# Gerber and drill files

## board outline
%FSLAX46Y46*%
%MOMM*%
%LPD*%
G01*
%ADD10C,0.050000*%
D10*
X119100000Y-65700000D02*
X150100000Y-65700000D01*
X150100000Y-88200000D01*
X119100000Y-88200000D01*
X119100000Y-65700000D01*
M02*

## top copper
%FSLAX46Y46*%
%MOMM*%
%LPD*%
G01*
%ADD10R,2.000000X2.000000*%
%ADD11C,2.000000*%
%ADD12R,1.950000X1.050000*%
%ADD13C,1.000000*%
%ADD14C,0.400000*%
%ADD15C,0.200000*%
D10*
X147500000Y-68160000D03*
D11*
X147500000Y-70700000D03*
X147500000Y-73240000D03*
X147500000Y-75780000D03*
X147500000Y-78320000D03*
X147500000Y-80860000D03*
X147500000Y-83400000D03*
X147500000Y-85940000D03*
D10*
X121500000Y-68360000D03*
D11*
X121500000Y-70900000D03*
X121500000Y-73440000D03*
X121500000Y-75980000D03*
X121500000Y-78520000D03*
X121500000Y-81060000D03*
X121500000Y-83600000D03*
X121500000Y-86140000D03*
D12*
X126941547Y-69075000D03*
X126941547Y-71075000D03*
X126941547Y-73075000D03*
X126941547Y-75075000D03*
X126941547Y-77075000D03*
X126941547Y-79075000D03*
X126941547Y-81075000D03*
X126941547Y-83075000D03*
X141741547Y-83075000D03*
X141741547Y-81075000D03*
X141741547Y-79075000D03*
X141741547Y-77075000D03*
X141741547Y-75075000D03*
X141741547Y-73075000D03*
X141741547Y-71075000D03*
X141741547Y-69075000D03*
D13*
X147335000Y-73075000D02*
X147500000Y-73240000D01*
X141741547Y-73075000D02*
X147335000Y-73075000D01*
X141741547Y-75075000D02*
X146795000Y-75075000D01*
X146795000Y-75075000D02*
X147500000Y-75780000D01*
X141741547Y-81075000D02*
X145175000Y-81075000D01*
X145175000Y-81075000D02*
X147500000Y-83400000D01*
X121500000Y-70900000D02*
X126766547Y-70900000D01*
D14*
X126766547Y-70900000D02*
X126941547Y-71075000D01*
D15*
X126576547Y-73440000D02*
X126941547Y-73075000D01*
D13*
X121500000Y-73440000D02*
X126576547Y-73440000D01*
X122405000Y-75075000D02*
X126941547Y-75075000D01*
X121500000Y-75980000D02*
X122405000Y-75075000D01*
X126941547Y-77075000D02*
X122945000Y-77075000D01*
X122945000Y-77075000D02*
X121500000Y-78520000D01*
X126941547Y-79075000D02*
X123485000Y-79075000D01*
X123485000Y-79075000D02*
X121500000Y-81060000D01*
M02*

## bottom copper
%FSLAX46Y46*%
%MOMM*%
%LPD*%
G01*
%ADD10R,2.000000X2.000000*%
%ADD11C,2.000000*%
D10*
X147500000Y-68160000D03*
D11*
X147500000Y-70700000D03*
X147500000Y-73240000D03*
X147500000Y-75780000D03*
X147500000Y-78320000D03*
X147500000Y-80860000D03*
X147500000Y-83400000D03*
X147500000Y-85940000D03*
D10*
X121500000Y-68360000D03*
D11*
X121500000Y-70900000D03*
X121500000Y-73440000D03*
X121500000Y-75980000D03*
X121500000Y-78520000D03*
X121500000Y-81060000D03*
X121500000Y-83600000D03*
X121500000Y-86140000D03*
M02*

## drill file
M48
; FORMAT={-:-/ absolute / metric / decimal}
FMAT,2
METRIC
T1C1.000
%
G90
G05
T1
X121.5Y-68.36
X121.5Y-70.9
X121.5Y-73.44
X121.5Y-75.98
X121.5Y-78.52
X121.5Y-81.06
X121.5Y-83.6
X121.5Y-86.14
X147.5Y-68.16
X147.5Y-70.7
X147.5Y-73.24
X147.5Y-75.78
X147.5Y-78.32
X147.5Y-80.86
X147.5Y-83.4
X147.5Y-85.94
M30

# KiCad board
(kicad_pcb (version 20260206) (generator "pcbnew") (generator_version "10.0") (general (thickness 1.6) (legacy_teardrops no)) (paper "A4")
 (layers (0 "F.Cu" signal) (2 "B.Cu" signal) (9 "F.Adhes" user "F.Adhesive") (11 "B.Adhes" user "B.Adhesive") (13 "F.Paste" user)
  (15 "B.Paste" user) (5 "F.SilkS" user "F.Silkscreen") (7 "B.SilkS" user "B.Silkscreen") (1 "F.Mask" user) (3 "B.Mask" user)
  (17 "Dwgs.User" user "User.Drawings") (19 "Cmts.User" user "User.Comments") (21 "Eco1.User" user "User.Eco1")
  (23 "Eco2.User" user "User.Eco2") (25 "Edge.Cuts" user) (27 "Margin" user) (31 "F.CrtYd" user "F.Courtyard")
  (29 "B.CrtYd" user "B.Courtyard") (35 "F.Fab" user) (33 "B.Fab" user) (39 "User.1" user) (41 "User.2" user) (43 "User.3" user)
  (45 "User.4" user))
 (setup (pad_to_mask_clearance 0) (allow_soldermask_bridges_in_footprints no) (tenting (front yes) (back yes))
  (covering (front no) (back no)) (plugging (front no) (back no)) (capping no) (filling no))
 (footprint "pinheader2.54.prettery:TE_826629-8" (layer "F.Cu") (at 147.5 68.16 -90)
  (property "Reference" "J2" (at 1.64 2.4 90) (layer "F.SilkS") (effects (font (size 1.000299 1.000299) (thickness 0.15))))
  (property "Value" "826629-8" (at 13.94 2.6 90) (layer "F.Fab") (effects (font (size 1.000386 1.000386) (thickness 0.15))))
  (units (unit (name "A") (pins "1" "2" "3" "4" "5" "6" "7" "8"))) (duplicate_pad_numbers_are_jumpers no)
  (pad "1" thru_hole rect (at 0 0 270) (size 2 2) (drill 1) (layers "*.Cu" "*.Mask") (remove_unused_layers no)
   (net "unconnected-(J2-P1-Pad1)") (solder_mask_margin 0.102))
  (pad "2" thru_hole circle (at 2.54 0 270) (size 2 2) (drill 1) (layers "*.Cu" "*.Mask") (remove_unused_layers no)
   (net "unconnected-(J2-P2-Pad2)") (solder_mask_margin 0.102))
  (pad "3" thru_hole circle (at 5.08 0 270) (size 2 2) (drill 1) (layers "*.Cu" "*.Mask") (remove_unused_layers no) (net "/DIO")
   (solder_mask_margin 0.102))
  (pad "4" thru_hole circle (at 7.62 0 270) (size 2 2) (drill 1) (layers "*.Cu" "*.Mask") (remove_unused_layers no) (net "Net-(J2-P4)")
   (solder_mask_margin 0.102))
  (pad "5" thru_hole circle (at 10.16 0 270) (size 2 2) (drill 1) (layers "*.Cu" "*.Mask") (remove_unused_layers no)
   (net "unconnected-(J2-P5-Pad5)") (solder_mask_margin 0.102))
  (pad "6" thru_hole circle (at 12.7 0 270) (size 2 2) (drill 1) (layers "*.Cu" "*.Mask") (remove_unused_layers no)
   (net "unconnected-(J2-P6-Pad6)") (solder_mask_margin 0.102))
  (pad "7" thru_hole circle (at 15.24 0 270) (size 2 2) (drill 1) (layers "*.Cu" "*.Mask") (remove_unused_layers no) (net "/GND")
   (solder_mask_margin 0.102))
  (pad "8" thru_hole circle (at 17.78 0 270) (size 2 2) (drill 1) (layers "*.Cu" "*.Mask") (remove_unused_layers no)
   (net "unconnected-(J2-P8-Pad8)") (solder_mask_margin 0.102)))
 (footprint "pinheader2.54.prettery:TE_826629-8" (layer "F.Cu") (at 121.5 68.36 -90)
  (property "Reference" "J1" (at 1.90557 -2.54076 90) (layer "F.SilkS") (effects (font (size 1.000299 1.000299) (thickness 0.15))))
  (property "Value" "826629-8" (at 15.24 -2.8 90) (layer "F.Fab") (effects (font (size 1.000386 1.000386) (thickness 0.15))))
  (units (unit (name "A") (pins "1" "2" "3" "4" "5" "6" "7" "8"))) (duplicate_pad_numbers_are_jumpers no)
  (pad "1" thru_hole rect (at 0 0 270) (size 2 2) (drill 1) (layers "*.Cu" "*.Mask") (remove_unused_layers no)
   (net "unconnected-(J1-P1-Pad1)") (solder_mask_margin 0.102) (thermal_gap 2)
   (teardrops (best_length_ratio 1.4) (max_length 1) (best_width_ratio 1) (max_width 0) (curved_edges no) (filter_ratio 0.9) (enabled no)
    (allow_two_segments yes) (prefer_zone_connections yes)))
  (pad "2" thru_hole circle (at 2.54 0 270) (size 2 2) (drill 1) (layers "*.Cu" "*.Mask") (remove_unused_layers no) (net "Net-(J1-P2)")
   (solder_mask_margin 0.102))
  (pad "3" thru_hole circle (at 5.08 0 270) (size 2 2) (drill 1) (layers "*.Cu" "*.Mask") (remove_unused_layers no) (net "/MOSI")
   (solder_mask_margin 0.102))
  (pad "4" thru_hole circle (at 7.62 0 270) (size 2 2) (drill 1) (layers "*.Cu" "*.Mask") (remove_unused_layers no) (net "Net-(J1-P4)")
   (solder_mask_margin 0.102))
  (pad "5" thru_hole circle (at 10.16 0 270) (size 2 2) (drill 1) (layers "*.Cu" "*.Mask") (remove_unused_layers no) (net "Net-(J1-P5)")
   (solder_mask_margin 0.102))
  (pad "6" thru_hole circle (at 12.7 0 270) (size 2 2) (drill 1) (layers "*.Cu" "*.Mask") (remove_unused_layers no) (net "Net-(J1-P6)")
   (solder_mask_margin 0.102))
  (pad "7" thru_hole circle (at 15.24 0 270) (size 2 2) (drill 1) (layers "*.Cu" "*.Mask") (remove_unused_layers no)
   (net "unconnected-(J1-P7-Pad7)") (solder_mask_margin 0.102))
  (pad "8" thru_hole circle (at 17.78 0 270) (size 2 2) (drill 1) (layers "*.Cu" "*.Mask") (remove_unused_layers no)
   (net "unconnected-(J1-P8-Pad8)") (solder_mask_margin 0.102)))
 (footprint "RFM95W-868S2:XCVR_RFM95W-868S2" (layer "F.Cu") (at 134.341547 76.075)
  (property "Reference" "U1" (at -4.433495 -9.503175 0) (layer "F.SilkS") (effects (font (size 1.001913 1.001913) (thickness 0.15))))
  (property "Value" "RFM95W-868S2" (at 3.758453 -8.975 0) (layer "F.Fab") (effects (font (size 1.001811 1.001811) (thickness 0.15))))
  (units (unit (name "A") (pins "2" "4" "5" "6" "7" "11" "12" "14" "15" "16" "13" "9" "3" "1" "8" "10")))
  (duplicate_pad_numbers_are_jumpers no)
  (pad "1" smd rect (at -7.4 -7) (size 1.95 1.05) (layers "F.Cu" "F.Mask" "F.Paste") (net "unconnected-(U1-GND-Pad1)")
   (solder_mask_margin 0.102))
  (pad "2" smd rect (at -7.4 -5) (size 1.95 1.05) (layers "F.Cu" "F.Mask" "F.Paste") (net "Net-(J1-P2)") (solder_mask_margin 0.102))
  (pad "3" smd rect (at -7.4 -3) (size 1.95 1.05) (layers "F.Cu" "F.Mask" "F.Paste") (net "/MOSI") (solder_mask_margin 0.102))
  (pad "4" smd rect (at -7.4 -1) (size 1.95 1.05) (layers "F.Cu" "F.Mask" "F.Paste") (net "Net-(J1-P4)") (solder_mask_margin 0.102))
  (pad "5" smd rect (at -7.4 1) (size 1.95 1.05) (layers "F.Cu" "F.Mask" "F.Paste") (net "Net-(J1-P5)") (solder_mask_margin 0.102))
  (pad "6" smd rect (at -7.4 3) (size 1.95 1.05) (layers "F.Cu" "F.Mask" "F.Paste") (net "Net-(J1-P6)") (solder_mask_margin 0.102))
  (pad "7" smd rect (at -7.4 5) (size 1.95 1.05) (layers "F.Cu" "F.Mask" "F.Paste") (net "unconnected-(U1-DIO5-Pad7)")
   (solder_mask_margin 0.102))
  (pad "8" smd rect (at -7.4 7) (size 1.95 1.05) (layers "F.Cu" "F.Mask" "F.Paste") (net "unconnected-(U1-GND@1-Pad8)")
   (solder_mask_margin 0.102))
  (pad "9" smd rect (at 7.4 7) (size 1.95 1.05) (layers "F.Cu" "F.Mask" "F.Paste") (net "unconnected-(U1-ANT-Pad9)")
   (solder_mask_margin 0.102))
  (pad "10" smd rect (at 7.4 5) (size 1.95 1.05) (layers "F.Cu" "F.Mask" "F.Paste") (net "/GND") (solder_mask_margin 0.102))
  (pad "11" smd rect (at 7.4 3) (size 1.95 1.05) (layers "F.Cu" "F.Mask" "F.Paste") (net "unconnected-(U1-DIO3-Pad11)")
   (solder_mask_margin 0.102))
  (pad "12" smd rect (at 7.4 1) (size 1.95 1.05) (layers "F.Cu" "F.Mask" "F.Paste") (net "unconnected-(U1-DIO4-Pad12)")
   (solder_mask_margin 0.102))
  (pad "13" smd rect (at 7.4 -1) (size 1.95 1.05) (layers "F.Cu" "F.Mask" "F.Paste") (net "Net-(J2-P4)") (solder_mask_margin 0.102))
  (pad "14" smd rect (at 7.4 -3) (size 1.95 1.05) (layers "F.Cu" "F.Mask" "F.Paste") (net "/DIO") (solder_mask_margin 0.102))
  (pad "15" smd rect (at 7.4 -5) (size 1.95 1.05) (layers "F.Cu" "F.Mask" "F.Paste") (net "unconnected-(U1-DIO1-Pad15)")
   (solder_mask_margin 0.102))
  (pad "16" smd rect (at 7.4 -7) (size 1.95 1.05) (layers "F.Cu" "F.Mask" "F.Paste") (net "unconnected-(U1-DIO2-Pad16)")
   (solder_mask_margin 0.102)))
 (gr_rect (start 119.1 65.7) (end 150.1 88.2) (stroke (width 0.05) (type default)) (fill no) (layer "Edge.Cuts"))
 (segment (start 147.335 73.075) (end 147.5 73.24) (width 1) (layer "F.Cu") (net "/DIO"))
 (segment (start 141.741547 73.075) (end 147.335 73.075) (width 1) (layer "F.Cu") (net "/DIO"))
 (segment (start 141.741547 75.075) (end 146.795 75.075) (width 1) (layer "F.Cu") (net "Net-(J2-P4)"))
 (segment (start 146.795 75.075) (end 147.5 75.78) (width 1) (layer "F.Cu") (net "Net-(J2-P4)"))
 (segment (start 141.741547 81.075) (end 145.175 81.075) (width 1) (layer "F.Cu") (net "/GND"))
 (segment (start 145.175 81.075) (end 147.5 83.4) (width 1) (layer "F.Cu") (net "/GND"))
 (segment (start 121.5 70.9) (end 126.766547 70.9) (width 1) (layer "F.Cu") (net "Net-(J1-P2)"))
 (segment (start 126.766547 70.9) (end 126.941547 71.075) (width 0.4) (layer "F.Cu") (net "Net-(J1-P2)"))
 (segment (start 126.576547 73.44) (end 126.941547 73.075) (width 0.2) (layer "F.Cu") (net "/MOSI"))
 (segment (start 121.5 73.44) (end 126.576547 73.44) (width 1) (layer "F.Cu") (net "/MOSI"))
 (segment (start 122.405 75.075) (end 126.941547 75.075) (width 1) (layer "F.Cu") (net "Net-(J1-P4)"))
 (segment (start 121.5 75.98) (end 122.405 75.075) (width 1) (layer "F.Cu") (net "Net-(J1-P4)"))
 (segment (start 126.941547 77.075) (end 122.945 77.075) (width 1) (layer "F.Cu") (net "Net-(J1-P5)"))
 (segment (start 122.945 77.075) (end 121.5 78.52) (width 1) (layer "F.Cu") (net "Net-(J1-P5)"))
 (segment (start 126.941547 79.075) (end 123.485 79.075) (width 1) (layer "F.Cu") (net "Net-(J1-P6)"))
 (segment (start 123.485 79.075) (end 121.5 81.06) (width 1) (layer "F.Cu") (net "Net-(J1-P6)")))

